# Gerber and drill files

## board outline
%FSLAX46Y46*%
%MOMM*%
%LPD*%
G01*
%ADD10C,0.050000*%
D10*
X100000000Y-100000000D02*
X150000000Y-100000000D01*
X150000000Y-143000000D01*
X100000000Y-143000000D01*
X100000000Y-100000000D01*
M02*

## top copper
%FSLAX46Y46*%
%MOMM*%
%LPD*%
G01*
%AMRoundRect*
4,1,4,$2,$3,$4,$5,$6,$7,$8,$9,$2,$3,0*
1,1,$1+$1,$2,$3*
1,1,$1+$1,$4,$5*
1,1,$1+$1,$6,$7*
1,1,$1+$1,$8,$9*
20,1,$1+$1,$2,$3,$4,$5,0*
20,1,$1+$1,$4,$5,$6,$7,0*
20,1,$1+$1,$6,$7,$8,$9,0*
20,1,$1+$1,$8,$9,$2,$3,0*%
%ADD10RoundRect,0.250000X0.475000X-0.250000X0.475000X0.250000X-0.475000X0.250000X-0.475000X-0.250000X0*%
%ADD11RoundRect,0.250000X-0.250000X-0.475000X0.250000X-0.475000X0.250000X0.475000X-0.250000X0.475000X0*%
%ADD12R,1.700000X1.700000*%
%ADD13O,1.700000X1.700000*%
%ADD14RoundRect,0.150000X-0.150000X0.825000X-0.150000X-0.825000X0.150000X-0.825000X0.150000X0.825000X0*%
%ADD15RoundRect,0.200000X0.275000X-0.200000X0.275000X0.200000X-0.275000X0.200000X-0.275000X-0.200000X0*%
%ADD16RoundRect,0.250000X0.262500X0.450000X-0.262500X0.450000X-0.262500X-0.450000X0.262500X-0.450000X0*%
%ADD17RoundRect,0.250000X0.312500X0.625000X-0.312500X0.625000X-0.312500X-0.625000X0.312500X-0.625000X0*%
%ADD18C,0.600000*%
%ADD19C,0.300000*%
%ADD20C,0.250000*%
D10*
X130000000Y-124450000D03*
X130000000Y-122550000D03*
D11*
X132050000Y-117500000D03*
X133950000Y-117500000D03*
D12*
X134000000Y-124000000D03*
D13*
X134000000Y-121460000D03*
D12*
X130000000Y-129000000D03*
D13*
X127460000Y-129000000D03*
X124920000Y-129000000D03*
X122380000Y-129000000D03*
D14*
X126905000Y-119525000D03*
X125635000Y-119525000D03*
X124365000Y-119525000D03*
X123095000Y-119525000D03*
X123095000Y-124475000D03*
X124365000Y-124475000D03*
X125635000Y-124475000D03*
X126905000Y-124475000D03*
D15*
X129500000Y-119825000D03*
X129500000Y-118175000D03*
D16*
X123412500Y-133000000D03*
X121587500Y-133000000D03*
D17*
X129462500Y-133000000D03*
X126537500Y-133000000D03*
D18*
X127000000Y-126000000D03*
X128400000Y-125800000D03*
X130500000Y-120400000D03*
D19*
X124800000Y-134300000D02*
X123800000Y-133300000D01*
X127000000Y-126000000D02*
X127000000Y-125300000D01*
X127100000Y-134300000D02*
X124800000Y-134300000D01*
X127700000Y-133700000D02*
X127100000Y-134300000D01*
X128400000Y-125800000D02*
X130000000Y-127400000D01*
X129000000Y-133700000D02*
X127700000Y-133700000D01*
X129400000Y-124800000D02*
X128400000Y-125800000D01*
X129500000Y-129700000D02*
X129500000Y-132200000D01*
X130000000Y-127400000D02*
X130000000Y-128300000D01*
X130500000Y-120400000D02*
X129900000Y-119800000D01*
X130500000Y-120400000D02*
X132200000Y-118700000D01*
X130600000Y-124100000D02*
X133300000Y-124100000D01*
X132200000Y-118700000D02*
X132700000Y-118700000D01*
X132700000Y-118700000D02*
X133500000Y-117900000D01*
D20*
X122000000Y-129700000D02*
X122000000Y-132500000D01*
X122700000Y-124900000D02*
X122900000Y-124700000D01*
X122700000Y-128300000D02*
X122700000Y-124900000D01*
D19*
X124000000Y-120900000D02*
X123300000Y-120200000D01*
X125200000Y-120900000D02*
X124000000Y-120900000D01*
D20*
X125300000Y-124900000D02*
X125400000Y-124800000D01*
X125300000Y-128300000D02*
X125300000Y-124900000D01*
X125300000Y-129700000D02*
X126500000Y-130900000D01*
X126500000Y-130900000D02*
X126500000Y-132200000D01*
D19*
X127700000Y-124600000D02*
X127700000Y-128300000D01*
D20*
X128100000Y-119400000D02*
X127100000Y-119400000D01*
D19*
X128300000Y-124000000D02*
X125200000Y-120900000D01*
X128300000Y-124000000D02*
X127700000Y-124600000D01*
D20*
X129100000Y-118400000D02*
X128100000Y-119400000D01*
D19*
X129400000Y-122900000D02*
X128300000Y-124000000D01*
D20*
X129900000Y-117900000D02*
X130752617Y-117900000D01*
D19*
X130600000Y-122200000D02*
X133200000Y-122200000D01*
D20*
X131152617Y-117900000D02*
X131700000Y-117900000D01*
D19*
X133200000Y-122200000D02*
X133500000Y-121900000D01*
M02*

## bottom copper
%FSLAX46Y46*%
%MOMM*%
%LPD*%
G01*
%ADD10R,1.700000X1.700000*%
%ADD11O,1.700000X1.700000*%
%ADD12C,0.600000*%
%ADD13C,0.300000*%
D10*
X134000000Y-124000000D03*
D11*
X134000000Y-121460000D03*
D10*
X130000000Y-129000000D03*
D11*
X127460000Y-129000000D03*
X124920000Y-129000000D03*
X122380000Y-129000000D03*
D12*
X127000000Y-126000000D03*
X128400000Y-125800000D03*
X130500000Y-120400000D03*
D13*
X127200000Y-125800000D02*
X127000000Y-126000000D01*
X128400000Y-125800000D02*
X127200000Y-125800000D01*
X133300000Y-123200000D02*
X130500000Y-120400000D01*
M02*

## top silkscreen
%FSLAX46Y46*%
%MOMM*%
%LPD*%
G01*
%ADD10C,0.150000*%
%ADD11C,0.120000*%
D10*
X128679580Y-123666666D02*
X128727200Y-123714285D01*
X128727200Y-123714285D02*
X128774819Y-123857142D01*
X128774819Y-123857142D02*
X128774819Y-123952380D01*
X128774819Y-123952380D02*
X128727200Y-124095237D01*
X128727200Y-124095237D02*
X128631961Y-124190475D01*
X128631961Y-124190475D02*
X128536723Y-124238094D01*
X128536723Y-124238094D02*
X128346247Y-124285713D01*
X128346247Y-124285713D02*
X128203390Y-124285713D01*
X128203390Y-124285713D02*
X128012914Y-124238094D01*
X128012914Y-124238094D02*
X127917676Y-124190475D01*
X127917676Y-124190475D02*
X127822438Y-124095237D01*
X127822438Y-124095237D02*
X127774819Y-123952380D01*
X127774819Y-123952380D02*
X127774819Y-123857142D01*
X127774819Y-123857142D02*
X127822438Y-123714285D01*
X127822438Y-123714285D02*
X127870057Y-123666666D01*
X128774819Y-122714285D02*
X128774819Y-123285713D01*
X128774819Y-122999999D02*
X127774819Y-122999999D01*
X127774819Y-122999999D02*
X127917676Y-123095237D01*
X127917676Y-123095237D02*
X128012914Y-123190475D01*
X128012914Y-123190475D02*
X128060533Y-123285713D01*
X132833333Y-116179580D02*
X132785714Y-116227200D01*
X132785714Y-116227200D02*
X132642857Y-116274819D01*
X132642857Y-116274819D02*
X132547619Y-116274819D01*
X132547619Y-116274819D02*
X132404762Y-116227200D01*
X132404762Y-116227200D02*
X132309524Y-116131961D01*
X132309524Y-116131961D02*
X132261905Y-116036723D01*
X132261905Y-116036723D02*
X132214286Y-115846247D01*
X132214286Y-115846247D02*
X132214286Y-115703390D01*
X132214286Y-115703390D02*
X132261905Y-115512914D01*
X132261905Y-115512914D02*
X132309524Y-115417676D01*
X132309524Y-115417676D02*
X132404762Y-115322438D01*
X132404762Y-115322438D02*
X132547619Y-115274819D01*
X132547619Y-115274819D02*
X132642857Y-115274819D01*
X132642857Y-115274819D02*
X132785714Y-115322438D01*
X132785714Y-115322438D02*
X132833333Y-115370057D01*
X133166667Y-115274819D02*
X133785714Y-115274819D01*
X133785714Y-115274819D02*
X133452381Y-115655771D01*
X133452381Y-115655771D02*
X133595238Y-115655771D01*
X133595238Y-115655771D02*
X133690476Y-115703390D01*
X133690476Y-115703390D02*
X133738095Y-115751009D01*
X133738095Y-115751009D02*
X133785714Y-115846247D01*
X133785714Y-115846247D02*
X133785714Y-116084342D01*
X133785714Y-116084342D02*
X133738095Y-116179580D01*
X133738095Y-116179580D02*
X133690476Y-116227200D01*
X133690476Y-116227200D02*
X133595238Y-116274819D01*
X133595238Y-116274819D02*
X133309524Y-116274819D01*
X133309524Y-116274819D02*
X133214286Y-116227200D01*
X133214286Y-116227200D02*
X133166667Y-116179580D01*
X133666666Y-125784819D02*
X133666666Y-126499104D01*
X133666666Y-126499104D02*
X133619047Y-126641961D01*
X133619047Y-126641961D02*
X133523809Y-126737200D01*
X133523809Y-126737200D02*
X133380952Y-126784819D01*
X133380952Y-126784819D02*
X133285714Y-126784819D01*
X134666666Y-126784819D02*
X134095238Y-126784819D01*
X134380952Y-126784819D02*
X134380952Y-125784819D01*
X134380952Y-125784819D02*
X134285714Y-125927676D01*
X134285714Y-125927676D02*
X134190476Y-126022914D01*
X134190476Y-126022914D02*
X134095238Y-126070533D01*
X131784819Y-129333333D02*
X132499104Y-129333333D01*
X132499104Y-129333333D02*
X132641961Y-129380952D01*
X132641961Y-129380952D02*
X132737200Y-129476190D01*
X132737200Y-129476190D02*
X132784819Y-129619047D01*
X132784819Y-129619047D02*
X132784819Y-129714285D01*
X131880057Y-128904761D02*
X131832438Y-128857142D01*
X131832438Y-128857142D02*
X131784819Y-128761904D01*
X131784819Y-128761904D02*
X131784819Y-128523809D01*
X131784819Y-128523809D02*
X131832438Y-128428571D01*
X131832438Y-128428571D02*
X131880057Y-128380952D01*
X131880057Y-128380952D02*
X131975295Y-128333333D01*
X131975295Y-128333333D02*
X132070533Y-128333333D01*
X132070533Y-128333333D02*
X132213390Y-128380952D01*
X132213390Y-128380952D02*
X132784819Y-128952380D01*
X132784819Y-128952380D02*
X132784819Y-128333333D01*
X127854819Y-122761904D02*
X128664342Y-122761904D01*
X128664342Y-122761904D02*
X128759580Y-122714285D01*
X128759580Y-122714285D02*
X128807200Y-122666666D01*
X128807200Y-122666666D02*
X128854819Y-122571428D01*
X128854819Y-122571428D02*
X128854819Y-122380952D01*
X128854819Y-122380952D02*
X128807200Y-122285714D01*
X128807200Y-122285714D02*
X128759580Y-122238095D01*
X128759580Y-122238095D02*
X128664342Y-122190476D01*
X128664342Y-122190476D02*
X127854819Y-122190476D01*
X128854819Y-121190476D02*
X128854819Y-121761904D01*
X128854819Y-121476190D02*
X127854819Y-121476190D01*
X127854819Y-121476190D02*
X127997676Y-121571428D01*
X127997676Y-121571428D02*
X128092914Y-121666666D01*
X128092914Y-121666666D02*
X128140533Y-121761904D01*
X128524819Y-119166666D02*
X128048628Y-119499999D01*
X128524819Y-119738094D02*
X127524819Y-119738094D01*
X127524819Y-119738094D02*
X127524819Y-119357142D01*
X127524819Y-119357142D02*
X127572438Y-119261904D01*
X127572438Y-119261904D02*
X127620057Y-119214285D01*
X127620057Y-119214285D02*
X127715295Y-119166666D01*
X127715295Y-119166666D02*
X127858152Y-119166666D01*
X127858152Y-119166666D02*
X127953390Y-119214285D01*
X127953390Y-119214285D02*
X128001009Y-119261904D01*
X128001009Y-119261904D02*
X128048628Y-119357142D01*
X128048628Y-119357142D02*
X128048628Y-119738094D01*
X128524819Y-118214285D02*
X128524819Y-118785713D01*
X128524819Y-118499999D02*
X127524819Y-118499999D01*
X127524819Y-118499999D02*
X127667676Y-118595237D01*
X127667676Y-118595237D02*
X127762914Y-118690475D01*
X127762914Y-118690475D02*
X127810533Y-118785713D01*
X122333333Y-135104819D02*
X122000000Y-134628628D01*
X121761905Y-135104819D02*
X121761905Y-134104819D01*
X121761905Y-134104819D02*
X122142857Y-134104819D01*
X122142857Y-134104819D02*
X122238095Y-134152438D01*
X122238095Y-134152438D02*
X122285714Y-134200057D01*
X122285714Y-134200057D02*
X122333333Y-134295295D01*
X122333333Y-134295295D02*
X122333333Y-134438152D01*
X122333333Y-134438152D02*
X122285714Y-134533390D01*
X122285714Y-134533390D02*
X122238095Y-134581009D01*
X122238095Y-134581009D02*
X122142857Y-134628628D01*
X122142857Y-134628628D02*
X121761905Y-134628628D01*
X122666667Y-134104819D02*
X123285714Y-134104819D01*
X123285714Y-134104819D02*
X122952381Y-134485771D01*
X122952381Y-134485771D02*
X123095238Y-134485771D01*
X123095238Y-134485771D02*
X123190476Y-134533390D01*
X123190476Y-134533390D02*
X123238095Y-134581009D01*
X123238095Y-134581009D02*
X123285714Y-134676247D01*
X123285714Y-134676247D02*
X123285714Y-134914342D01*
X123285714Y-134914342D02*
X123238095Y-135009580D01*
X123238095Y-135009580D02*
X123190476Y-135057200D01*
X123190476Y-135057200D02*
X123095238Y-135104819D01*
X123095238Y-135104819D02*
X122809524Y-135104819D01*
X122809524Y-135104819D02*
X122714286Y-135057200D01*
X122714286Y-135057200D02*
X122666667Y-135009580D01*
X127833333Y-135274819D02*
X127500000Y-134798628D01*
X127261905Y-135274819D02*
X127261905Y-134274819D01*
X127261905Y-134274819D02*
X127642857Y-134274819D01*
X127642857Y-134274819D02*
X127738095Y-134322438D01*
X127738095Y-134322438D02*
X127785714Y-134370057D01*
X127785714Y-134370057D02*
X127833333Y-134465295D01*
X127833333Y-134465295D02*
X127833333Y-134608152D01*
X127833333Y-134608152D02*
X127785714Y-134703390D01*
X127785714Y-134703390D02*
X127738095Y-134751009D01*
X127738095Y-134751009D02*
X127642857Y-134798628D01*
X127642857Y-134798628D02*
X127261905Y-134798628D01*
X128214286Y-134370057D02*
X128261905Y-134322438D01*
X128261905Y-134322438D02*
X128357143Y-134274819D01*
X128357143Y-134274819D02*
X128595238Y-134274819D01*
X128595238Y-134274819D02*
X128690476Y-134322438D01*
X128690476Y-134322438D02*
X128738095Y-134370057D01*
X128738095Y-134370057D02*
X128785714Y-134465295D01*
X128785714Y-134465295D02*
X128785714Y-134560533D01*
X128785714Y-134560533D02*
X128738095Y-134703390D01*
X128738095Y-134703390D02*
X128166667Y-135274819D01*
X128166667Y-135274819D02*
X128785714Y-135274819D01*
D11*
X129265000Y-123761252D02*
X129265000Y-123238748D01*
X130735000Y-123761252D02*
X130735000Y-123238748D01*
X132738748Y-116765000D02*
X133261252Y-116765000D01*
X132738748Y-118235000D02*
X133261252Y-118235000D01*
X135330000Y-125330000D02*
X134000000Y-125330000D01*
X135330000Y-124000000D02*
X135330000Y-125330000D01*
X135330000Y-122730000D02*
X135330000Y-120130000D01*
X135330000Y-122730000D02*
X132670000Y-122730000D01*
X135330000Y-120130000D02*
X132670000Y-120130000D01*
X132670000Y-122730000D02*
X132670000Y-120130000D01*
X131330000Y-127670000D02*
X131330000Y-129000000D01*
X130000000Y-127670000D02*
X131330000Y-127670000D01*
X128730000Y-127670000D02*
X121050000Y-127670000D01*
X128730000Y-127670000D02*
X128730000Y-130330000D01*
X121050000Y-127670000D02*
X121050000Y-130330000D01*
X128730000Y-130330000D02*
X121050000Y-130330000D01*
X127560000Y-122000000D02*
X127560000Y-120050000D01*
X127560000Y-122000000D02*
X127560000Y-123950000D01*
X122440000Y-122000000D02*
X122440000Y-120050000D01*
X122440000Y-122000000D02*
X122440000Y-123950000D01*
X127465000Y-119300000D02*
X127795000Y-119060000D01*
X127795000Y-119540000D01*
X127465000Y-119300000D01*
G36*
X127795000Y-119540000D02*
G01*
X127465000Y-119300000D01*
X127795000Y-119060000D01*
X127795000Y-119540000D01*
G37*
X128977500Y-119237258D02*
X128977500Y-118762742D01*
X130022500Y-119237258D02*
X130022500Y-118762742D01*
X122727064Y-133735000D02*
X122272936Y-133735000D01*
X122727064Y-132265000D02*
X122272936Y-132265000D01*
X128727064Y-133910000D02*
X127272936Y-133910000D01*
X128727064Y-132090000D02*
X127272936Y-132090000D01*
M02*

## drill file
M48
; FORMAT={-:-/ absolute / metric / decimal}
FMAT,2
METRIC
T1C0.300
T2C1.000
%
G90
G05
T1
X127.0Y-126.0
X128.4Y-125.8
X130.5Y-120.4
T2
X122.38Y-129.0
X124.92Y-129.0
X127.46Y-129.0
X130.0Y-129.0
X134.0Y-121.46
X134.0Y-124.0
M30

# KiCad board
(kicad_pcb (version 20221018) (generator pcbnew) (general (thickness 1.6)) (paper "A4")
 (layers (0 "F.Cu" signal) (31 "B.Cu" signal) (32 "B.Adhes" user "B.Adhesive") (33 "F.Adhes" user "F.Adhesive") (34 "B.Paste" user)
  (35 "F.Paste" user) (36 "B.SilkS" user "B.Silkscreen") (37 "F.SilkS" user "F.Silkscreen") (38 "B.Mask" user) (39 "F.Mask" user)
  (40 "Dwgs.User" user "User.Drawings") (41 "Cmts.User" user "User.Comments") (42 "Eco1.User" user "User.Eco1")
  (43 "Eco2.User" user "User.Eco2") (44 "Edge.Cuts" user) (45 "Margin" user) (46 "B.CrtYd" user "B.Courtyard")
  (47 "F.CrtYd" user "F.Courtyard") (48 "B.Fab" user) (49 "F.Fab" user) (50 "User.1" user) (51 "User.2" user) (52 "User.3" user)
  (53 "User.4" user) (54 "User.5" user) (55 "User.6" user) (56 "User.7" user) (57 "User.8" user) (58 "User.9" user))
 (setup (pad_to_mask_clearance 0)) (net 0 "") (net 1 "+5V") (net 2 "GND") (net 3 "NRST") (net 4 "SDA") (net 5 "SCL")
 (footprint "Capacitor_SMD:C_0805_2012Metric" (layer "F.Cu") (at 130 123.5 90)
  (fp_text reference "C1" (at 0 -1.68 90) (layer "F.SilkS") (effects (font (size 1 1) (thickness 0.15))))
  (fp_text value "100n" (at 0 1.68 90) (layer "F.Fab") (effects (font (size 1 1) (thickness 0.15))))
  (fp_line (start -0.261252 -0.735) (end 0.261252 -0.735) (stroke (width 0.12) (type solid)) (layer "F.SilkS"))
  (fp_line (start -0.261252 0.735) (end 0.261252 0.735) (stroke (width 0.12) (type solid)) (layer "F.SilkS"))
  (pad "1" smd roundrect (at -0.95 0 90) (size 1 1.45) (layers "F.Cu" "F.Paste" "F.Mask") (roundrect_rratio 0.25) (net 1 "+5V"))
  (pad "2" smd roundrect (at 0.95 0 90) (size 1 1.45) (layers "F.Cu" "F.Paste" "F.Mask") (roundrect_rratio 0.25) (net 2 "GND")))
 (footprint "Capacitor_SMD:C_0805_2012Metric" (layer "F.Cu") (at 133 117.5)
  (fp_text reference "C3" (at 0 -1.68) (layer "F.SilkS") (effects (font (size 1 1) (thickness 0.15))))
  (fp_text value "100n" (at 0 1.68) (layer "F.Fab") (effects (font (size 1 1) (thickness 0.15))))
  (fp_line (start -0.261252 -0.735) (end 0.261252 -0.735) (stroke (width 0.12) (type solid)) (layer "F.SilkS"))
  (fp_line (start -0.261252 0.735) (end 0.261252 0.735) (stroke (width 0.12) (type solid)) (layer "F.SilkS"))
  (pad "1" smd roundrect (at -0.95 0) (size 1 1.45) (layers "F.Cu" "F.Paste" "F.Mask") (roundrect_rratio 0.25) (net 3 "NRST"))
  (pad "2" smd roundrect (at 0.95 0) (size 1 1.45) (layers "F.Cu" "F.Paste" "F.Mask") (roundrect_rratio 0.25) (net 1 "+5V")))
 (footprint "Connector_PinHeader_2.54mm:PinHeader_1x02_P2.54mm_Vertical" (layer "F.Cu") (at 134 124 180)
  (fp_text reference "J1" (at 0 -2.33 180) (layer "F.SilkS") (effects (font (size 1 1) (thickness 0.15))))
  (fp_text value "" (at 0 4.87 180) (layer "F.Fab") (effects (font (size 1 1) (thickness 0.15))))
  (fp_line (start -1.33 -1.33) (end 0 -1.33) (stroke (width 0.12) (type solid)) (layer "F.SilkS"))
  (fp_line (start -1.33 0) (end -1.33 -1.33) (stroke (width 0.12) (type solid)) (layer "F.SilkS"))
  (fp_line (start -1.33 1.27) (end -1.33 3.87) (stroke (width 0.12) (type solid)) (layer "F.SilkS"))
  (fp_line (start -1.33 1.27) (end 1.33 1.27) (stroke (width 0.12) (type solid)) (layer "F.SilkS"))
  (fp_line (start -1.33 3.87) (end 1.33 3.87) (stroke (width 0.12) (type solid)) (layer "F.SilkS"))
  (fp_line (start 1.33 1.27) (end 1.33 3.87) (stroke (width 0.12) (type solid)) (layer "F.SilkS"))
  (pad "1" thru_hole rect (at 0 0 180) (size 1.7 1.7) (drill 1) (layers "*.Cu" "*.Mask") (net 1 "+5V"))
  (pad "2" thru_hole oval (at 0 2.54 180) (size 1.7 1.7) (drill 1) (layers "*.Cu" "*.Mask") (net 2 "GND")))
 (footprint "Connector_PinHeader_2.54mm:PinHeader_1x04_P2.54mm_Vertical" (layer "F.Cu") (at 130 129 -90)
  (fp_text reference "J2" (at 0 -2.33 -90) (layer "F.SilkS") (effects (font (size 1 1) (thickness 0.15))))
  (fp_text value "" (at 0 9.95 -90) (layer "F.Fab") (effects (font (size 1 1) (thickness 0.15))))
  (fp_line (start -1.33 -1.33) (end 0 -1.33) (stroke (width 0.12) (type solid)) (layer "F.SilkS"))
  (fp_line (start -1.33 0) (end -1.33 -1.33) (stroke (width 0.12) (type solid)) (layer "F.SilkS"))
  (fp_line (start -1.33 1.27) (end -1.33 8.95) (stroke (width 0.12) (type solid)) (layer "F.SilkS"))
  (fp_line (start -1.33 1.27) (end 1.33 1.27) (stroke (width 0.12) (type solid)) (layer "F.SilkS"))
  (fp_line (start -1.33 8.95) (end 1.33 8.95) (stroke (width 0.12) (type solid)) (layer "F.SilkS"))
  (fp_line (start 1.33 1.27) (end 1.33 8.95) (stroke (width 0.12) (type solid)) (layer "F.SilkS"))
  (pad "1" thru_hole rect (at 0 0 270) (size 1.7 1.7) (drill 1) (layers "*.Cu" "*.Mask") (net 1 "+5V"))
  (pad "2" thru_hole oval (at 0 2.54 270) (size 1.7 1.7) (drill 1) (layers "*.Cu" "*.Mask") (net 2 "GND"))
  (pad "3" thru_hole oval (at 0 5.08 270) (size 1.7 1.7) (drill 1) (layers "*.Cu" "*.Mask") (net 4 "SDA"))
  (pad "4" thru_hole oval (at 0 7.62 270) (size 1.7 1.7) (drill 1) (layers "*.Cu" "*.Mask") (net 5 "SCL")))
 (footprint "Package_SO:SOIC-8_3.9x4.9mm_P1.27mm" (layer "F.Cu") (at 125 122 -90)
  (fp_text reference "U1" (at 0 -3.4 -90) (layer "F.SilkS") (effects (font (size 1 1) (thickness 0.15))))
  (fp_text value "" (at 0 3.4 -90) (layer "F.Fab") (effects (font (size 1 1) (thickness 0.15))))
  (fp_line (start 0 -2.56) (end -1.95 -2.56) (stroke (width 0.12) (type solid)) (layer "F.SilkS"))
  (fp_line (start 0 -2.56) (end 1.95 -2.56) (stroke (width 0.12) (type solid)) (layer "F.SilkS"))
  (fp_line (start 0 2.56) (end -1.95 2.56) (stroke (width 0.12) (type solid)) (layer "F.SilkS"))
  (fp_line (start 0 2.56) (end 1.95 2.56) (stroke (width 0.12) (type solid)) (layer "F.SilkS"))
  (fp_poly
   (pts (xy -2.7 -2.465) (xy -2.94 -2.795) (xy -2.46 -2.795) (xy -2.7 -2.465)) (stroke (width 0.12) (type solid)) (fill solid)
   (layer "F.SilkS"))
  (pad "1" smd roundrect (at -2.475 -1.905 270) (size 1.95 0.6) (layers "F.Cu" "F.Paste" "F.Mask") (roundrect_rratio 0.25) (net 3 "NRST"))
  (pad "2" smd roundrect (at -2.475 -0.635 270) (size 1.95 0.6) (layers "F.Cu" "F.Paste" "F.Mask") (roundrect_rratio 0.25))
  (pad "3" smd roundrect (at -2.475 0.635 270) (size 1.95 0.6) (layers "F.Cu" "F.Paste" "F.Mask") (roundrect_rratio 0.25))
  (pad "4" smd roundrect (at -2.475 1.905 270) (size 1.95 0.6) (layers "F.Cu" "F.Paste" "F.Mask") (roundrect_rratio 0.25) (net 2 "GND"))
  (pad "5" smd roundrect (at 2.475 1.905 270) (size 1.95 0.6) (layers "F.Cu" "F.Paste" "F.Mask") (roundrect_rratio 0.25) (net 5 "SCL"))
  (pad "6" smd roundrect (at 2.475 0.635 270) (size 1.95 0.6) (layers "F.Cu" "F.Paste" "F.Mask") (roundrect_rratio 0.25))
  (pad "7" smd roundrect (at 2.475 -0.635 270) (size 1.95 0.6) (layers "F.Cu" "F.Paste" "F.Mask") (roundrect_rratio 0.25) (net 4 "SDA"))
  (pad "8" smd roundrect (at 2.475 -1.905 270) (size 1.95 0.6) (layers "F.Cu" "F.Paste" "F.Mask") (roundrect_rratio 0.25) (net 1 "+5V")))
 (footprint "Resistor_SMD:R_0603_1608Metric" (layer "F.Cu") (at 129.5 119 90)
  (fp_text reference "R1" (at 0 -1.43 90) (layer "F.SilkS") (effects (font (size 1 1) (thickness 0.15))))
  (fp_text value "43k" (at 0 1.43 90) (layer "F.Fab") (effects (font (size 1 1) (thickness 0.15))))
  (fp_line (start -0.237258 -0.5225) (end 0.237258 -0.5225) (stroke (width 0.12) (type solid)) (layer "F.SilkS"))
  (fp_line (start -0.237258 0.5225) (end 0.237258 0.5225) (stroke (width 0.12) (type solid)) (layer "F.SilkS"))
  (pad "1" smd roundrect (at -0.825 0 90) (size 0.8 0.95) (layers "F.Cu" "F.Paste" "F.Mask") (roundrect_rratio 0.25) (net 1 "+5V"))
  (pad "2" smd roundrect (at 0.825 0 90) (size 0.8 0.95) (layers "F.Cu" "F.Paste" "F.Mask") (roundrect_rratio 0.25) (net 3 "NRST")))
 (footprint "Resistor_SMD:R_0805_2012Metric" (layer "F.Cu") (at 122.5 133 180)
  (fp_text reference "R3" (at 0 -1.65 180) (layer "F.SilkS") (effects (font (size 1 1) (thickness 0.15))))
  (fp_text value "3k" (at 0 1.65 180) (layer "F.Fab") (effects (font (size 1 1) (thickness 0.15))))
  (fp_line (start -0.227064 -0.735) (end 0.227064 -0.735) (stroke (width 0.12) (type solid)) (layer "F.SilkS"))
  (fp_line (start -0.227064 0.735) (end 0.227064 0.735) (stroke (width 0.12) (type solid)) (layer "F.SilkS"))
  (pad "1" smd roundrect (at -0.9125 0 180) (size 1.025 1.4) (layers "F.Cu" "F.Paste" "F.Mask") (roundrect_rratio 0.243902) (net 1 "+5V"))
  (pad "2" smd roundrect (at 0.9125 0 180) (size 1.025 1.4) (layers "F.Cu" "F.Paste" "F.Mask") (roundrect_rratio 0.243902) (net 5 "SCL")))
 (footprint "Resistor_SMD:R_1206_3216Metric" (layer "F.Cu") (at 128 133 180)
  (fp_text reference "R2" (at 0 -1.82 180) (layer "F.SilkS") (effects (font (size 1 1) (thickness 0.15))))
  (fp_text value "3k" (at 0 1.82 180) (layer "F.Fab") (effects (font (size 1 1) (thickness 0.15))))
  (fp_line (start -0.727064 -0.91) (end 0.727064 -0.91) (stroke (width 0.12) (type solid)) (layer "F.SilkS"))
  (fp_line (start -0.727064 0.91) (end 0.727064 0.91) (stroke (width 0.12) (type solid)) (layer "F.SilkS"))
  (pad "1" smd roundrect (at -1.4625 0 180) (size 1.125 1.75) (layers "F.Cu" "F.Paste" "F.Mask") (roundrect_rratio 0.222222) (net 1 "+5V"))
  (pad "2" smd roundrect (at 1.4625 0 180) (size 1.125 1.75) (layers "F.Cu" "F.Paste" "F.Mask") (roundrect_rratio 0.222222) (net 4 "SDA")))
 (gr_rect (start 100 100) (end 150 143) (stroke (width 0.05) (type default)) (fill none) (layer "Edge.Cuts"))
 (segment (start 124.8 134.3) (end 123.8 133.3) (width 0.3) (layer "F.Cu") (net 1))
 (segment (start 127 126) (end 127 125.3) (width 0.3) (layer "F.Cu") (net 1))
 (segment (start 127.1 134.3) (end 124.8 134.3) (width 0.3) (layer "F.Cu") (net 1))
 (segment (start 127.7 133.7) (end 127.1 134.3) (width 0.3) (layer "F.Cu") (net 1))
 (segment (start 128.4 125.8) (end 130 127.4) (width 0.3) (layer "F.Cu") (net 1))
 (segment (start 129 133.7) (end 127.7 133.7) (width 0.3) (layer "F.Cu") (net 1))
 (segment (start 129.4 124.8) (end 128.4 125.8) (width 0.3) (layer "F.Cu") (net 1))
 (segment (start 129.5 129.7) (end 129.5 132.2) (width 0.3) (layer "F.Cu") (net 1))
 (segment (start 130 127.4) (end 130 128.3) (width 0.3) (layer "F.Cu") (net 1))
 (segment (start 130.5 120.4) (end 129.9 119.8) (width 0.3) (layer "F.Cu") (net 1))
 (segment (start 130.5 120.4) (end 132.2 118.7) (width 0.3) (layer "F.Cu") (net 1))
 (segment (start 130.6 124.1) (end 133.3 124.1) (width 0.3) (layer "F.Cu") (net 1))
 (segment (start 132.2 118.7) (end 132.7 118.7) (width 0.3) (layer "F.Cu") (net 1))
 (segment (start 132.7 118.7) (end 133.5 117.9) (width 0.3) (layer "F.Cu") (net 1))
 (via (at 127 126) (size 0.6) (drill 0.3) (layers "F.Cu" "B.Cu") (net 1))
 (via (at 128.4 125.8) (size 0.6) (drill 0.3) (layers "F.Cu" "B.Cu") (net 1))
 (via (at 130.5 120.4) (size 0.6) (drill 0.3) (layers "F.Cu" "B.Cu") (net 1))
 (segment (start 122 129.7) (end 122 132.5) (width 0.25) (layer "F.Cu") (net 5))
 (segment (start 122.7 124.9) (end 122.9 124.7) (width 0.25) (layer "F.Cu") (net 5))
 (segment (start 122.7 128.3) (end 122.7 124.9) (width 0.25) (layer "F.Cu") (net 5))
 (segment (start 124 120.9) (end 123.3 120.2) (width 0.3) (layer "F.Cu") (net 2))
 (segment (start 125.2 120.9) (end 124 120.9) (width 0.3) (layer "F.Cu") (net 2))
 (segment (start 125.3 124.9) (end 125.4 124.8) (width 0.25) (layer "F.Cu") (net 4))
 (segment (start 125.3 128.3) (end 125.3 124.9) (width 0.25) (layer "F.Cu") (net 4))
 (segment (start 125.3 129.7) (end 126.5 130.9) (width 0.25) (layer "F.Cu") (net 4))
 (segment (start 126.5 130.9) (end 126.5 132.2) (width 0.25) (layer "F.Cu") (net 4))
 (segment (start 127.2 125.8) (end 127 126) (width 0.3) (layer "B.Cu") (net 1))
 (segment (start 127.7 124.6) (end 127.7 128.3) (width 0.3) (layer "F.Cu") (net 2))
 (segment (start 128.1 119.4) (end 127.1 119.4) (width 0.25) (layer "F.Cu") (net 3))
 (segment (start 128.3 124) (end 125.2 120.9) (width 0.3) (layer "F.Cu") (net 2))
 (segment (start 128.3 124) (end 127.7 124.6) (width 0.3) (layer "F.Cu") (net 2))
 (segment (start 128.4 125.8) (end 127.2 125.8) (width 0.3) (layer "B.Cu") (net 1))
 (segment (start 129.1 118.4) (end 128.1 119.4) (width 0.25) (layer "F.Cu") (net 3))
 (segment (start 129.4 122.9) (end 128.3 124) (width 0.3) (layer "F.Cu") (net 2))
 (segment (start 129.9 117.9) (end 130.752617 117.9) (width 0.25) (layer "F.Cu") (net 3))
 (segment (start 130.6 122.2) (end 133.2 122.2) (width 0.3) (layer "F.Cu") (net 2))
 (segment (start 131.152617 117.9) (end 131.7 117.9) (width 0.25) (layer "F.Cu") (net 3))
 (segment (start 133.2 122.2) (end 133.5 121.9) (width 0.3) (layer "F.Cu") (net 2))
 (segment (start 133.3 123.2) (end 130.5 120.4) (width 0.3) (layer "B.Cu") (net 1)))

